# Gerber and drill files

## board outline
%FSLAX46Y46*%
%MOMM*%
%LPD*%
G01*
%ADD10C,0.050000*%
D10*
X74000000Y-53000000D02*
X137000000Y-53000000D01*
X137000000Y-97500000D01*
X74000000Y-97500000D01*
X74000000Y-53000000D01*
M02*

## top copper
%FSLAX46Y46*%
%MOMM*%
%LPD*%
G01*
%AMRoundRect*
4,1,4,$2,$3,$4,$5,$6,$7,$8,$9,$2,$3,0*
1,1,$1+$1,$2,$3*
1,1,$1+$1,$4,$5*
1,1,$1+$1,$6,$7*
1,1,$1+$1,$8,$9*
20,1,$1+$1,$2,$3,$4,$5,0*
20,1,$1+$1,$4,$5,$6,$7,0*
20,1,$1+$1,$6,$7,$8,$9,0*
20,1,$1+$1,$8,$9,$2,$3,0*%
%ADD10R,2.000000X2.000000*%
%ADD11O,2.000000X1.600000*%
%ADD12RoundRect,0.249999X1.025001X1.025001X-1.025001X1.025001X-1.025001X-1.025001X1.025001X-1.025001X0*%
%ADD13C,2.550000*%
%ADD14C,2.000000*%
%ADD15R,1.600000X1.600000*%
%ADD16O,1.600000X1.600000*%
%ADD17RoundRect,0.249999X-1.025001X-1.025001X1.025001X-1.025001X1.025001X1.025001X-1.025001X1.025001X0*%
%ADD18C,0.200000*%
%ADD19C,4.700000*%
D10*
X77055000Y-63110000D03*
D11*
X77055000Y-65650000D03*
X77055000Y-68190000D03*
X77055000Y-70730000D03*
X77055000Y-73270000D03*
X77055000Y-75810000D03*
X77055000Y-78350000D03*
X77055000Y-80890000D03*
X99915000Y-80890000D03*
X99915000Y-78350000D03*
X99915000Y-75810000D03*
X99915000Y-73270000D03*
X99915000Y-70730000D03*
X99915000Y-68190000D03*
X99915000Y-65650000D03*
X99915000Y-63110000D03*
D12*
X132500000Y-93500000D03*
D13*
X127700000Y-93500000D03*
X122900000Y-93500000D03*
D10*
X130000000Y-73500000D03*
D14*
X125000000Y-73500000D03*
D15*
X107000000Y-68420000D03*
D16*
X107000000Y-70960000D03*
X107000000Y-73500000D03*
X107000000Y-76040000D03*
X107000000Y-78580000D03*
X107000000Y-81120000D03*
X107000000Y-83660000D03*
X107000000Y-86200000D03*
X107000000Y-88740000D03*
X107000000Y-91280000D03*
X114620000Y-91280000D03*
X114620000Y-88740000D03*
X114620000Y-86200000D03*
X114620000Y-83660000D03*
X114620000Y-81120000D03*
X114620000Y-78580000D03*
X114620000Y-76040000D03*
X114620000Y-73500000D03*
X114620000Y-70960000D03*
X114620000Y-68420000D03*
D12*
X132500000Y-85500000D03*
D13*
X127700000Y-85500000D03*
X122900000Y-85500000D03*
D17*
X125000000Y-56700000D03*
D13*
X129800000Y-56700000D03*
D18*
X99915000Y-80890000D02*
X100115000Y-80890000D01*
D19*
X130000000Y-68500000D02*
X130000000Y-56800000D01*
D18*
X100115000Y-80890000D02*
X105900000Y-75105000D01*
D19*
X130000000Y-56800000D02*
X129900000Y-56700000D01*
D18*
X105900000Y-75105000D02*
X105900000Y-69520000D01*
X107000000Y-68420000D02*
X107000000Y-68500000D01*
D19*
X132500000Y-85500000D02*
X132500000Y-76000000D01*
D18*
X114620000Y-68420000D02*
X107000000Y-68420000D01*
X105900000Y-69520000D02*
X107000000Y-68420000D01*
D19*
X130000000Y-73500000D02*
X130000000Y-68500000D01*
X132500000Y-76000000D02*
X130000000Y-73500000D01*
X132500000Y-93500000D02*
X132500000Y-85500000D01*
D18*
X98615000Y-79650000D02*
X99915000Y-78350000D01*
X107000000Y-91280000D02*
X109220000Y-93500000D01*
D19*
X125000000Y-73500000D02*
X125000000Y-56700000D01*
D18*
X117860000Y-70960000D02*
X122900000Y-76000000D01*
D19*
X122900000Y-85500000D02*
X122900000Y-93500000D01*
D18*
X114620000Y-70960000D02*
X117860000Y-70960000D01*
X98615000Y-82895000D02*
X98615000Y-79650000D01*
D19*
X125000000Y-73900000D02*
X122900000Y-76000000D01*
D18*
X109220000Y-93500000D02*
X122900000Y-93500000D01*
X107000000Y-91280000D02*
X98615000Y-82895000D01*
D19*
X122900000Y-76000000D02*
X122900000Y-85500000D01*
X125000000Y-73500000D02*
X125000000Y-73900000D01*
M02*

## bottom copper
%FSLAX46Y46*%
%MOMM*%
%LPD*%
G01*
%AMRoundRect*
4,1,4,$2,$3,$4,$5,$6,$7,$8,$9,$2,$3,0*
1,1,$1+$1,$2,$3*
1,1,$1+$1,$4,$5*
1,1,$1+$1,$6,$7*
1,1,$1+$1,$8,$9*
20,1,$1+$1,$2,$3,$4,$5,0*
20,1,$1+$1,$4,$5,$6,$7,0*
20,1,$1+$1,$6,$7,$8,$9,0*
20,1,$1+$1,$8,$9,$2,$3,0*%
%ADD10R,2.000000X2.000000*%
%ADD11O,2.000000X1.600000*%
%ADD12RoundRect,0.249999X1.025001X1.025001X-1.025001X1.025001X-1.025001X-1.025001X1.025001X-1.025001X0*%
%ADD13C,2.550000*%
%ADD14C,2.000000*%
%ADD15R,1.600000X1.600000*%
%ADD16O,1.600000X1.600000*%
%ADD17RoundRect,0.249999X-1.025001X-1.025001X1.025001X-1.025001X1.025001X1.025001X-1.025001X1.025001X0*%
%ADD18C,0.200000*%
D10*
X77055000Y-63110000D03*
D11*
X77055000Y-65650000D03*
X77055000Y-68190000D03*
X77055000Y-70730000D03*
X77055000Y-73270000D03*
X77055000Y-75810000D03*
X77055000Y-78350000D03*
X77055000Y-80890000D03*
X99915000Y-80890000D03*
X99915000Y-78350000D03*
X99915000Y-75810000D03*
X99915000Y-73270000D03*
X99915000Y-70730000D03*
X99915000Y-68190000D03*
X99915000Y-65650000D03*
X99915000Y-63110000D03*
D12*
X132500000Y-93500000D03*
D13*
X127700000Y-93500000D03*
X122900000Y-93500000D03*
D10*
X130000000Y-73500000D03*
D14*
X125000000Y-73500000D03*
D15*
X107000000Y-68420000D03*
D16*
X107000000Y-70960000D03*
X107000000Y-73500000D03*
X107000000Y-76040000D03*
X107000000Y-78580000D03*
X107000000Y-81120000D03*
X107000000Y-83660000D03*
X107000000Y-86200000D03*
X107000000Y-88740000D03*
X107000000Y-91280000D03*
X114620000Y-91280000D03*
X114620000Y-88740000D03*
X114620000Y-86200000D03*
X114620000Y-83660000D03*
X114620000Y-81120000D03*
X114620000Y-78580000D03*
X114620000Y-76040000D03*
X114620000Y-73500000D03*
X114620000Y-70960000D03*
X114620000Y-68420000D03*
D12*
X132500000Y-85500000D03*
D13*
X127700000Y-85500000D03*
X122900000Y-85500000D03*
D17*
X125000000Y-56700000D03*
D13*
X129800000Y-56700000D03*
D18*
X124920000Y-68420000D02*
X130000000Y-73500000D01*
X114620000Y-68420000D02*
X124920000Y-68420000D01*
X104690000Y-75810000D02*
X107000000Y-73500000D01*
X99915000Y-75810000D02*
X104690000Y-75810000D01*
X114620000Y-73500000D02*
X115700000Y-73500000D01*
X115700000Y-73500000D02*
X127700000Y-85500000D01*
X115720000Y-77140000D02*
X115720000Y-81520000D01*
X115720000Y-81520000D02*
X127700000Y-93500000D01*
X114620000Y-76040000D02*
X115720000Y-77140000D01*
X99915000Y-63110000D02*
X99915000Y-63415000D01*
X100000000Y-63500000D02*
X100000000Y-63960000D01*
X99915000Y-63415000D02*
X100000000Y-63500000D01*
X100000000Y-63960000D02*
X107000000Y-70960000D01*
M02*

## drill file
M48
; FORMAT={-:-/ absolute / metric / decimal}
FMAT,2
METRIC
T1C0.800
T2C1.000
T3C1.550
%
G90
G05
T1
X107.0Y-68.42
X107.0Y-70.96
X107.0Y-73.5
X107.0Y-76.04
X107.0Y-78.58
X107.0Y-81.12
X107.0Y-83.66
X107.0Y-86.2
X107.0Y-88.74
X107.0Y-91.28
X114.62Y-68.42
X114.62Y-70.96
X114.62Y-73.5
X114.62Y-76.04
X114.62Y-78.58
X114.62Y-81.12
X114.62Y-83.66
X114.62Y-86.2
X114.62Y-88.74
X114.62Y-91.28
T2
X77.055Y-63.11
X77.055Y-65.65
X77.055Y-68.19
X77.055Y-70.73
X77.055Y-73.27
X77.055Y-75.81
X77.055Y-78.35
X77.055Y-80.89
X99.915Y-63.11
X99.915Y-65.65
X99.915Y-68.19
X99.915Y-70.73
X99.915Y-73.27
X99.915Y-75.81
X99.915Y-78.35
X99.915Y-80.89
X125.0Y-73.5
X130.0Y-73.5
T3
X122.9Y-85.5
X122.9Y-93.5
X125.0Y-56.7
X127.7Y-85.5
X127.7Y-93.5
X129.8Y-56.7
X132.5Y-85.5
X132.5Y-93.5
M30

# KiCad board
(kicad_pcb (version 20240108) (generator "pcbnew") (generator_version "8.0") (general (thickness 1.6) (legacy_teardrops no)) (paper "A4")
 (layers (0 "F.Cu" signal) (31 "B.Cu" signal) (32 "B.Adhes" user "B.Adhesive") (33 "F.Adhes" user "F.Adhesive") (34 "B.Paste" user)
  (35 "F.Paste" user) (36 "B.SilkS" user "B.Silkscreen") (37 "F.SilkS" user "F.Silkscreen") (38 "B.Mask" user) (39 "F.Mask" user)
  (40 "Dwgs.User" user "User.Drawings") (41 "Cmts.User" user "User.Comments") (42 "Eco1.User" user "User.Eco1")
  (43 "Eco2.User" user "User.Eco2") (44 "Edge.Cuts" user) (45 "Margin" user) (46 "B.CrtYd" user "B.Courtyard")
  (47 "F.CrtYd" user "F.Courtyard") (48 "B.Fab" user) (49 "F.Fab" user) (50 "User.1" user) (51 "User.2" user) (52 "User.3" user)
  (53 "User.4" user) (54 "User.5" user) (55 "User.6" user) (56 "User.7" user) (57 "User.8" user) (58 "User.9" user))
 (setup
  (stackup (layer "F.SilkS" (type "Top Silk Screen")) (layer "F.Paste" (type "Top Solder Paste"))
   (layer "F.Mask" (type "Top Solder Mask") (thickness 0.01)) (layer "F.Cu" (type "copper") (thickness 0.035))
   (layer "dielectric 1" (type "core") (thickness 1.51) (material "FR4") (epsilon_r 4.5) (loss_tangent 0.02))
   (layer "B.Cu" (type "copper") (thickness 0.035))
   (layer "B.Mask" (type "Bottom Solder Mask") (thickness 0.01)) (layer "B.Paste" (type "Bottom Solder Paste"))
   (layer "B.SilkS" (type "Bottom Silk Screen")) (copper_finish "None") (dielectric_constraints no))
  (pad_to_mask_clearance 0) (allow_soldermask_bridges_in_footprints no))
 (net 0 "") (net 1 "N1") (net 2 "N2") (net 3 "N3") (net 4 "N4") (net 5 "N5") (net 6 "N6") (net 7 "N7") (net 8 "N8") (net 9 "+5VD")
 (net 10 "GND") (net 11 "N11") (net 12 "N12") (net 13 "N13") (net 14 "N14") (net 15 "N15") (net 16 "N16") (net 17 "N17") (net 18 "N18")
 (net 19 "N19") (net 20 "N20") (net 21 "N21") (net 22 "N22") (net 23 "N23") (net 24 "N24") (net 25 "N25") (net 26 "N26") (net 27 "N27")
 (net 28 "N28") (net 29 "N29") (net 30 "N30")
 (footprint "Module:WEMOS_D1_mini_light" (layer "F.Cu") (at 77.055 63.11)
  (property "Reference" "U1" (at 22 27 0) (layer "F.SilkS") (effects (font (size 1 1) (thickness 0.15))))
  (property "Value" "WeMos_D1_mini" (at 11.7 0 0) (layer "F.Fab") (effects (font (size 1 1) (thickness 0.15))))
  (pad "1" thru_hole rect (at 0 0) (size 2 2) (drill 1) (layers "*.Cu" "*.Mask") (remove_unused_layers no) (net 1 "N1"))
  (pad "2" thru_hole oval (at 0 2.54) (size 2 1.6) (drill 1) (layers "*.Cu" "*.Mask") (remove_unused_layers no) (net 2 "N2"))
  (pad "3" thru_hole oval (at 0 5.08) (size 2 1.6) (drill 1) (layers "*.Cu" "*.Mask") (remove_unused_layers no) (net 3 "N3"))
  (pad "4" thru_hole oval (at 0 7.62) (size 2 1.6) (drill 1) (layers "*.Cu" "*.Mask") (remove_unused_layers no) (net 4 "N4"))
  (pad "5" thru_hole oval (at 0 10.16) (size 2 1.6) (drill 1) (layers "*.Cu" "*.Mask") (remove_unused_layers no) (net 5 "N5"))
  (pad "6" thru_hole oval (at 0 12.7) (size 2 1.6) (drill 1) (layers "*.Cu" "*.Mask") (remove_unused_layers no) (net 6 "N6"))
  (pad "7" thru_hole oval (at 0 15.24) (size 2 1.6) (drill 1) (layers "*.Cu" "*.Mask") (remove_unused_layers no) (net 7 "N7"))
  (pad "8" thru_hole oval (at 0 17.78) (size 2 1.6) (drill 1) (layers "*.Cu" "*.Mask") (remove_unused_layers no) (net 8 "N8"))
  (pad "9" thru_hole oval (at 22.86 17.78) (size 2 1.6) (drill 1) (layers "*.Cu" "*.Mask") (remove_unused_layers no) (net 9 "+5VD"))
  (pad "10" thru_hole oval (at 22.86 15.24) (size 2 1.6) (drill 1) (layers "*.Cu" "*.Mask") (remove_unused_layers no) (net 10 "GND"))
  (pad "11" thru_hole oval (at 22.86 12.7) (size 2 1.6) (drill 1) (layers "*.Cu" "*.Mask") (remove_unused_layers no) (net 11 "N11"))
  (pad "12" thru_hole oval (at 22.86 10.16) (size 2 1.6) (drill 1) (layers "*.Cu" "*.Mask") (remove_unused_layers no) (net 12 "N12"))
  (pad "13" thru_hole oval (at 22.86 7.62) (size 2 1.6) (drill 1) (layers "*.Cu" "*.Mask") (remove_unused_layers no) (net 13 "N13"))
  (pad "14" thru_hole oval (at 22.86 5.08) (size 2 1.6) (drill 1) (layers "*.Cu" "*.Mask") (remove_unused_layers no) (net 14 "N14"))
  (pad "15" thru_hole oval (at 22.86 2.54) (size 2 1.6) (drill 1) (layers "*.Cu" "*.Mask") (remove_unused_layers no) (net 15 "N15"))
  (pad "16" thru_hole oval (at 22.86 0) (size 2 1.6) (drill 1) (layers "*.Cu" "*.Mask") (remove_unused_layers no) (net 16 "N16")))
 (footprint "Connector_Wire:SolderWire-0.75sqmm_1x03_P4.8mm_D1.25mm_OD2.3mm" (layer "F.Cu") (at 132.5 93.5 180)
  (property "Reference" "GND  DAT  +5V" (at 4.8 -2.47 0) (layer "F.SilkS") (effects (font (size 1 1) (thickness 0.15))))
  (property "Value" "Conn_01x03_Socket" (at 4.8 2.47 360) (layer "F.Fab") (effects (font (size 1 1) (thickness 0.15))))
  (pad "1" thru_hole roundrect (at 0 0 180) (size 2.55 2.55) (drill 1.55) (layers "*.Cu" "*.Mask") (remove_unused_layers no)
   (roundrect_rratio 0.098039) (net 9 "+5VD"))
  (pad "2" thru_hole circle (at 4.8 0 180) (size 2.55 2.55) (drill 1.55) (layers "*.Cu" "*.Mask") (remove_unused_layers no) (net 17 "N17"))
  (pad "3" thru_hole circle (at 9.6 0 180) (size 2.55 2.55) (drill 1.55) (layers "*.Cu" "*.Mask") (remove_unused_layers no) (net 10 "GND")))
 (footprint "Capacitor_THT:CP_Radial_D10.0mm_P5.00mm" (layer "F.Cu") (at 130 73.5 180)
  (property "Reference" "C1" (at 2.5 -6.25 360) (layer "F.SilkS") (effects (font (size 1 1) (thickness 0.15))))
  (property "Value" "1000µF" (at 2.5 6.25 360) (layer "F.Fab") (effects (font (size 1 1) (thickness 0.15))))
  (pad "1" thru_hole rect (at 0 0 180) (size 2 2) (drill 1) (layers "*.Cu" "*.Mask") (remove_unused_layers no) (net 9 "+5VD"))
  (pad "2" thru_hole circle (at 5 0 180) (size 2 2) (drill 1) (layers "*.Cu" "*.Mask") (remove_unused_layers no) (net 10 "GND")))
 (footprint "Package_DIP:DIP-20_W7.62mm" (layer "F.Cu") (at 107 68.42)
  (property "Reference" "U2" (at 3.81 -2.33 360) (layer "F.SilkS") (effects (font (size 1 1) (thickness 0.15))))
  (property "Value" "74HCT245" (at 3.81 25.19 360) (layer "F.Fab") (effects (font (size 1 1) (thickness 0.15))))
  (pad "1" thru_hole rect (at 0 0) (size 1.6 1.6) (drill 0.8) (layers "*.Cu" "*.Mask") (remove_unused_layers no) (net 9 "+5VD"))
  (pad "2" thru_hole oval (at 0 2.54) (size 1.6 1.6) (drill 0.8) (layers "*.Cu" "*.Mask") (remove_unused_layers no) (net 16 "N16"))
  (pad "3" thru_hole oval (at 0 5.08) (size 1.6 1.6) (drill 0.8) (layers "*.Cu" "*.Mask") (remove_unused_layers no) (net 11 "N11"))
  (pad "4" thru_hole oval (at 0 7.62) (size 1.6 1.6) (drill 0.8) (layers "*.Cu" "*.Mask") (remove_unused_layers no) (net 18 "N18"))
  (pad "5" thru_hole oval (at 0 10.16) (size 1.6 1.6) (drill 0.8) (layers "*.Cu" "*.Mask") (remove_unused_layers no) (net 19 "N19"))
  (pad "6" thru_hole oval (at 0 12.7) (size 1.6 1.6) (drill 0.8) (layers "*.Cu" "*.Mask") (remove_unused_layers no) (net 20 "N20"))
  (pad "7" thru_hole oval (at 0 15.24) (size 1.6 1.6) (drill 0.8) (layers "*.Cu" "*.Mask") (remove_unused_layers no) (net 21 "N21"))
  (pad "8" thru_hole oval (at 0 17.78) (size 1.6 1.6) (drill 0.8) (layers "*.Cu" "*.Mask") (remove_unused_layers no) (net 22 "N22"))
  (pad "9" thru_hole oval (at 0 20.32) (size 1.6 1.6) (drill 0.8) (layers "*.Cu" "*.Mask") (remove_unused_layers no) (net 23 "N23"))
  (pad "10" thru_hole oval (at 0 22.86) (size 1.6 1.6) (drill 0.8) (layers "*.Cu" "*.Mask") (remove_unused_layers no) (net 10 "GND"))
  (pad "11" thru_hole oval (at 7.62 22.86) (size 1.6 1.6) (drill 0.8) (layers "*.Cu" "*.Mask") (remove_unused_layers no) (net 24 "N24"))
  (pad "12" thru_hole oval (at 7.62 20.32) (size 1.6 1.6) (drill 0.8) (layers "*.Cu" "*.Mask") (remove_unused_layers no) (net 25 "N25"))
  (pad "13" thru_hole oval (at 7.62 17.78) (size 1.6 1.6) (drill 0.8) (layers "*.Cu" "*.Mask") (remove_unused_layers no) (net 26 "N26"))
  (pad "14" thru_hole oval (at 7.62 15.24) (size 1.6 1.6) (drill 0.8) (layers "*.Cu" "*.Mask") (remove_unused_layers no) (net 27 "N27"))
  (pad "15" thru_hole oval (at 7.62 12.7) (size 1.6 1.6) (drill 0.8) (layers "*.Cu" "*.Mask") (remove_unused_layers no) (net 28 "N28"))
  (pad "16" thru_hole oval (at 7.62 10.16) (size 1.6 1.6) (drill 0.8) (layers "*.Cu" "*.Mask") (remove_unused_layers no) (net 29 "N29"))
  (pad "17" thru_hole oval (at 7.62 7.62) (size 1.6 1.6) (drill 0.8) (layers "*.Cu" "*.Mask") (remove_unused_layers no) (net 17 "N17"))
  (pad "18" thru_hole oval (at 7.62 5.08) (size 1.6 1.6) (drill 0.8) (layers "*.Cu" "*.Mask") (remove_unused_layers no) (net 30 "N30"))
  (pad "19" thru_hole oval (at 7.62 2.54) (size 1.6 1.6) (drill 0.8) (layers "*.Cu" "*.Mask") (remove_unused_layers no) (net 10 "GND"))
  (pad "20" thru_hole oval (at 7.62 0) (size 1.6 1.6) (drill 0.8) (layers "*.Cu" "*.Mask") (remove_unused_layers no) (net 9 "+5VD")))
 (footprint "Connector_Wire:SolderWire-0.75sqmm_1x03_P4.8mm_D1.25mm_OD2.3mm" (layer "F.Cu") (at 132.5 85.5 180)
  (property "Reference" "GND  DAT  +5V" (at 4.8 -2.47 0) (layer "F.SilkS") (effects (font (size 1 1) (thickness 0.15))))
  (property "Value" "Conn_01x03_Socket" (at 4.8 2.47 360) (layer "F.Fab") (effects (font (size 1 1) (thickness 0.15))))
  (pad "1" thru_hole roundrect (at 0 0 180) (size 2.55 2.55) (drill 1.55) (layers "*.Cu" "*.Mask") (remove_unused_layers no)
   (roundrect_rratio 0.098039) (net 9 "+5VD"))
  (pad "2" thru_hole circle (at 4.8 0 180) (size 2.55 2.55) (drill 1.55) (layers "*.Cu" "*.Mask") (remove_unused_layers no) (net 30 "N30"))
  (pad "3" thru_hole circle (at 9.6 0 180) (size 2.55 2.55) (drill 1.55) (layers "*.Cu" "*.Mask") (remove_unused_layers no) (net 10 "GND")))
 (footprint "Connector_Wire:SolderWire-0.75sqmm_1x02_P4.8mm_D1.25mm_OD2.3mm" (layer "F.Cu") (at 125 56.7)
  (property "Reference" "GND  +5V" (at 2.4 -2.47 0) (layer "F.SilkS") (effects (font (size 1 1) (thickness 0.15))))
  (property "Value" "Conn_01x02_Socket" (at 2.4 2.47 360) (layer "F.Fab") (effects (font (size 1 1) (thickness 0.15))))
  (pad "1" thru_hole roundrect (at 0 0) (size 2.55 2.55) (drill 1.55) (layers "*.Cu" "*.Mask") (remove_unused_layers no)
   (roundrect_rratio 0.098039) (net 10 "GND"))
  (pad "2" thru_hole circle (at 4.8 0) (size 2.55 2.55) (drill 1.55) (layers "*.Cu" "*.Mask") (remove_unused_layers no) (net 9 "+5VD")))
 (gr_rect (start 74 53) (end 137 97.5) (stroke (width 0.05) (type default)) (fill none) (layer "Edge.Cuts"))
 (segment (start 99.915 80.89) (end 100.115 80.89) (width 0.2) (layer "F.Cu") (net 9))
 (segment (start 130 68.5) (end 130 56.8) (width 4.7) (layer "F.Cu") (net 9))
 (segment (start 100.115 80.89) (end 105.9 75.105) (width 0.2) (layer "F.Cu") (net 9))
 (segment (start 130 56.8) (end 129.9 56.7) (width 4.7) (layer "F.Cu") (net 9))
 (segment (start 105.9 75.105) (end 105.9 69.52) (width 0.2) (layer "F.Cu") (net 9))
 (segment (start 107 68.42) (end 107 68.5) (width 0.2) (layer "F.Cu") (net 9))
 (segment (start 132.5 85.5) (end 132.5 76) (width 4.7) (layer "F.Cu") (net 9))
 (segment (start 114.62 68.42) (end 107 68.42) (width 0.2) (layer "F.Cu") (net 9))
 (segment (start 105.9 69.52) (end 107 68.42) (width 0.2) (layer "F.Cu") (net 9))
 (segment (start 130 73.5) (end 130 68.5) (width 4.7) (layer "F.Cu") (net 9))
 (segment (start 132.5 76) (end 130 73.5) (width 4.7) (layer "F.Cu") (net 9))
 (segment (start 132.5 93.5) (end 132.5 85.5) (width 4.7) (layer "F.Cu") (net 9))
 (segment (start 124.92 68.42) (end 130 73.5) (width 0.2) (layer "B.Cu") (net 9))
 (segment (start 114.62 68.42) (end 124.92 68.42) (width 0.2) (layer "B.Cu") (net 9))
 (segment (start 98.615 79.65) (end 99.915 78.35) (width 0.2) (layer "F.Cu") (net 10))
 (segment (start 107 91.28) (end 109.22 93.5) (width 0.2) (layer "F.Cu") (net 10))
 (segment (start 125 73.5) (end 125 56.7) (width 4.7) (layer "F.Cu") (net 10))
 (segment (start 117.86 70.96) (end 122.9 76) (width 0.2) (layer "F.Cu") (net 10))
 (segment (start 122.9 85.5) (end 122.9 93.5) (width 4.7) (layer "F.Cu") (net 10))
 (segment (start 114.62 70.96) (end 117.86 70.96) (width 0.2) (layer "F.Cu") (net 10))
 (segment (start 98.615 82.895) (end 98.615 79.65) (width 0.2) (layer "F.Cu") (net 10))
 (segment (start 125 73.9) (end 122.9 76) (width 4.7) (layer "F.Cu") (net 10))
 (segment (start 109.22 93.5) (end 122.9 93.5) (width 0.2) (layer "F.Cu") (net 10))
 (segment (start 107 91.28) (end 98.615 82.895) (width 0.2) (layer "F.Cu") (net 10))
 (segment (start 122.9 76) (end 122.9 85.5) (width 4.7) (layer "F.Cu") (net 10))
 (segment (start 125 73.5) (end 125 73.9) (width 4.7) (layer "F.Cu") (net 10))
 (segment (start 104.69 75.81) (end 107 73.5) (width 0.2) (layer "B.Cu") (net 11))
 (segment (start 99.915 75.81) (end 104.69 75.81) (width 0.2) (layer "B.Cu") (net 11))
 (segment (start 114.62 73.5) (end 115.7 73.5) (width 0.2) (layer "B.Cu") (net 30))
 (segment (start 115.7 73.5) (end 127.7 85.5) (width 0.2) (layer "B.Cu") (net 30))
 (segment (start 115.72 77.14) (end 115.72 81.52) (width 0.2) (layer "B.Cu") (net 17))
 (segment (start 115.72 81.52) (end 127.7 93.5) (width 0.2) (layer "B.Cu") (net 17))
 (segment (start 114.62 76.04) (end 115.72 77.14) (width 0.2) (layer "B.Cu") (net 17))
 (segment (start 99.915 63.11) (end 99.915 63.415) (width 0.2) (layer "B.Cu") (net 16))
 (segment (start 100 63.5) (end 100 63.96) (width 0.2) (layer "B.Cu") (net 16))
 (segment (start 99.915 63.415) (end 100 63.5) (width 0.2) (layer "B.Cu") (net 16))
 (segment (start 100 63.96) (end 107 70.96) (width 0.2) (layer "B.Cu") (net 16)))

